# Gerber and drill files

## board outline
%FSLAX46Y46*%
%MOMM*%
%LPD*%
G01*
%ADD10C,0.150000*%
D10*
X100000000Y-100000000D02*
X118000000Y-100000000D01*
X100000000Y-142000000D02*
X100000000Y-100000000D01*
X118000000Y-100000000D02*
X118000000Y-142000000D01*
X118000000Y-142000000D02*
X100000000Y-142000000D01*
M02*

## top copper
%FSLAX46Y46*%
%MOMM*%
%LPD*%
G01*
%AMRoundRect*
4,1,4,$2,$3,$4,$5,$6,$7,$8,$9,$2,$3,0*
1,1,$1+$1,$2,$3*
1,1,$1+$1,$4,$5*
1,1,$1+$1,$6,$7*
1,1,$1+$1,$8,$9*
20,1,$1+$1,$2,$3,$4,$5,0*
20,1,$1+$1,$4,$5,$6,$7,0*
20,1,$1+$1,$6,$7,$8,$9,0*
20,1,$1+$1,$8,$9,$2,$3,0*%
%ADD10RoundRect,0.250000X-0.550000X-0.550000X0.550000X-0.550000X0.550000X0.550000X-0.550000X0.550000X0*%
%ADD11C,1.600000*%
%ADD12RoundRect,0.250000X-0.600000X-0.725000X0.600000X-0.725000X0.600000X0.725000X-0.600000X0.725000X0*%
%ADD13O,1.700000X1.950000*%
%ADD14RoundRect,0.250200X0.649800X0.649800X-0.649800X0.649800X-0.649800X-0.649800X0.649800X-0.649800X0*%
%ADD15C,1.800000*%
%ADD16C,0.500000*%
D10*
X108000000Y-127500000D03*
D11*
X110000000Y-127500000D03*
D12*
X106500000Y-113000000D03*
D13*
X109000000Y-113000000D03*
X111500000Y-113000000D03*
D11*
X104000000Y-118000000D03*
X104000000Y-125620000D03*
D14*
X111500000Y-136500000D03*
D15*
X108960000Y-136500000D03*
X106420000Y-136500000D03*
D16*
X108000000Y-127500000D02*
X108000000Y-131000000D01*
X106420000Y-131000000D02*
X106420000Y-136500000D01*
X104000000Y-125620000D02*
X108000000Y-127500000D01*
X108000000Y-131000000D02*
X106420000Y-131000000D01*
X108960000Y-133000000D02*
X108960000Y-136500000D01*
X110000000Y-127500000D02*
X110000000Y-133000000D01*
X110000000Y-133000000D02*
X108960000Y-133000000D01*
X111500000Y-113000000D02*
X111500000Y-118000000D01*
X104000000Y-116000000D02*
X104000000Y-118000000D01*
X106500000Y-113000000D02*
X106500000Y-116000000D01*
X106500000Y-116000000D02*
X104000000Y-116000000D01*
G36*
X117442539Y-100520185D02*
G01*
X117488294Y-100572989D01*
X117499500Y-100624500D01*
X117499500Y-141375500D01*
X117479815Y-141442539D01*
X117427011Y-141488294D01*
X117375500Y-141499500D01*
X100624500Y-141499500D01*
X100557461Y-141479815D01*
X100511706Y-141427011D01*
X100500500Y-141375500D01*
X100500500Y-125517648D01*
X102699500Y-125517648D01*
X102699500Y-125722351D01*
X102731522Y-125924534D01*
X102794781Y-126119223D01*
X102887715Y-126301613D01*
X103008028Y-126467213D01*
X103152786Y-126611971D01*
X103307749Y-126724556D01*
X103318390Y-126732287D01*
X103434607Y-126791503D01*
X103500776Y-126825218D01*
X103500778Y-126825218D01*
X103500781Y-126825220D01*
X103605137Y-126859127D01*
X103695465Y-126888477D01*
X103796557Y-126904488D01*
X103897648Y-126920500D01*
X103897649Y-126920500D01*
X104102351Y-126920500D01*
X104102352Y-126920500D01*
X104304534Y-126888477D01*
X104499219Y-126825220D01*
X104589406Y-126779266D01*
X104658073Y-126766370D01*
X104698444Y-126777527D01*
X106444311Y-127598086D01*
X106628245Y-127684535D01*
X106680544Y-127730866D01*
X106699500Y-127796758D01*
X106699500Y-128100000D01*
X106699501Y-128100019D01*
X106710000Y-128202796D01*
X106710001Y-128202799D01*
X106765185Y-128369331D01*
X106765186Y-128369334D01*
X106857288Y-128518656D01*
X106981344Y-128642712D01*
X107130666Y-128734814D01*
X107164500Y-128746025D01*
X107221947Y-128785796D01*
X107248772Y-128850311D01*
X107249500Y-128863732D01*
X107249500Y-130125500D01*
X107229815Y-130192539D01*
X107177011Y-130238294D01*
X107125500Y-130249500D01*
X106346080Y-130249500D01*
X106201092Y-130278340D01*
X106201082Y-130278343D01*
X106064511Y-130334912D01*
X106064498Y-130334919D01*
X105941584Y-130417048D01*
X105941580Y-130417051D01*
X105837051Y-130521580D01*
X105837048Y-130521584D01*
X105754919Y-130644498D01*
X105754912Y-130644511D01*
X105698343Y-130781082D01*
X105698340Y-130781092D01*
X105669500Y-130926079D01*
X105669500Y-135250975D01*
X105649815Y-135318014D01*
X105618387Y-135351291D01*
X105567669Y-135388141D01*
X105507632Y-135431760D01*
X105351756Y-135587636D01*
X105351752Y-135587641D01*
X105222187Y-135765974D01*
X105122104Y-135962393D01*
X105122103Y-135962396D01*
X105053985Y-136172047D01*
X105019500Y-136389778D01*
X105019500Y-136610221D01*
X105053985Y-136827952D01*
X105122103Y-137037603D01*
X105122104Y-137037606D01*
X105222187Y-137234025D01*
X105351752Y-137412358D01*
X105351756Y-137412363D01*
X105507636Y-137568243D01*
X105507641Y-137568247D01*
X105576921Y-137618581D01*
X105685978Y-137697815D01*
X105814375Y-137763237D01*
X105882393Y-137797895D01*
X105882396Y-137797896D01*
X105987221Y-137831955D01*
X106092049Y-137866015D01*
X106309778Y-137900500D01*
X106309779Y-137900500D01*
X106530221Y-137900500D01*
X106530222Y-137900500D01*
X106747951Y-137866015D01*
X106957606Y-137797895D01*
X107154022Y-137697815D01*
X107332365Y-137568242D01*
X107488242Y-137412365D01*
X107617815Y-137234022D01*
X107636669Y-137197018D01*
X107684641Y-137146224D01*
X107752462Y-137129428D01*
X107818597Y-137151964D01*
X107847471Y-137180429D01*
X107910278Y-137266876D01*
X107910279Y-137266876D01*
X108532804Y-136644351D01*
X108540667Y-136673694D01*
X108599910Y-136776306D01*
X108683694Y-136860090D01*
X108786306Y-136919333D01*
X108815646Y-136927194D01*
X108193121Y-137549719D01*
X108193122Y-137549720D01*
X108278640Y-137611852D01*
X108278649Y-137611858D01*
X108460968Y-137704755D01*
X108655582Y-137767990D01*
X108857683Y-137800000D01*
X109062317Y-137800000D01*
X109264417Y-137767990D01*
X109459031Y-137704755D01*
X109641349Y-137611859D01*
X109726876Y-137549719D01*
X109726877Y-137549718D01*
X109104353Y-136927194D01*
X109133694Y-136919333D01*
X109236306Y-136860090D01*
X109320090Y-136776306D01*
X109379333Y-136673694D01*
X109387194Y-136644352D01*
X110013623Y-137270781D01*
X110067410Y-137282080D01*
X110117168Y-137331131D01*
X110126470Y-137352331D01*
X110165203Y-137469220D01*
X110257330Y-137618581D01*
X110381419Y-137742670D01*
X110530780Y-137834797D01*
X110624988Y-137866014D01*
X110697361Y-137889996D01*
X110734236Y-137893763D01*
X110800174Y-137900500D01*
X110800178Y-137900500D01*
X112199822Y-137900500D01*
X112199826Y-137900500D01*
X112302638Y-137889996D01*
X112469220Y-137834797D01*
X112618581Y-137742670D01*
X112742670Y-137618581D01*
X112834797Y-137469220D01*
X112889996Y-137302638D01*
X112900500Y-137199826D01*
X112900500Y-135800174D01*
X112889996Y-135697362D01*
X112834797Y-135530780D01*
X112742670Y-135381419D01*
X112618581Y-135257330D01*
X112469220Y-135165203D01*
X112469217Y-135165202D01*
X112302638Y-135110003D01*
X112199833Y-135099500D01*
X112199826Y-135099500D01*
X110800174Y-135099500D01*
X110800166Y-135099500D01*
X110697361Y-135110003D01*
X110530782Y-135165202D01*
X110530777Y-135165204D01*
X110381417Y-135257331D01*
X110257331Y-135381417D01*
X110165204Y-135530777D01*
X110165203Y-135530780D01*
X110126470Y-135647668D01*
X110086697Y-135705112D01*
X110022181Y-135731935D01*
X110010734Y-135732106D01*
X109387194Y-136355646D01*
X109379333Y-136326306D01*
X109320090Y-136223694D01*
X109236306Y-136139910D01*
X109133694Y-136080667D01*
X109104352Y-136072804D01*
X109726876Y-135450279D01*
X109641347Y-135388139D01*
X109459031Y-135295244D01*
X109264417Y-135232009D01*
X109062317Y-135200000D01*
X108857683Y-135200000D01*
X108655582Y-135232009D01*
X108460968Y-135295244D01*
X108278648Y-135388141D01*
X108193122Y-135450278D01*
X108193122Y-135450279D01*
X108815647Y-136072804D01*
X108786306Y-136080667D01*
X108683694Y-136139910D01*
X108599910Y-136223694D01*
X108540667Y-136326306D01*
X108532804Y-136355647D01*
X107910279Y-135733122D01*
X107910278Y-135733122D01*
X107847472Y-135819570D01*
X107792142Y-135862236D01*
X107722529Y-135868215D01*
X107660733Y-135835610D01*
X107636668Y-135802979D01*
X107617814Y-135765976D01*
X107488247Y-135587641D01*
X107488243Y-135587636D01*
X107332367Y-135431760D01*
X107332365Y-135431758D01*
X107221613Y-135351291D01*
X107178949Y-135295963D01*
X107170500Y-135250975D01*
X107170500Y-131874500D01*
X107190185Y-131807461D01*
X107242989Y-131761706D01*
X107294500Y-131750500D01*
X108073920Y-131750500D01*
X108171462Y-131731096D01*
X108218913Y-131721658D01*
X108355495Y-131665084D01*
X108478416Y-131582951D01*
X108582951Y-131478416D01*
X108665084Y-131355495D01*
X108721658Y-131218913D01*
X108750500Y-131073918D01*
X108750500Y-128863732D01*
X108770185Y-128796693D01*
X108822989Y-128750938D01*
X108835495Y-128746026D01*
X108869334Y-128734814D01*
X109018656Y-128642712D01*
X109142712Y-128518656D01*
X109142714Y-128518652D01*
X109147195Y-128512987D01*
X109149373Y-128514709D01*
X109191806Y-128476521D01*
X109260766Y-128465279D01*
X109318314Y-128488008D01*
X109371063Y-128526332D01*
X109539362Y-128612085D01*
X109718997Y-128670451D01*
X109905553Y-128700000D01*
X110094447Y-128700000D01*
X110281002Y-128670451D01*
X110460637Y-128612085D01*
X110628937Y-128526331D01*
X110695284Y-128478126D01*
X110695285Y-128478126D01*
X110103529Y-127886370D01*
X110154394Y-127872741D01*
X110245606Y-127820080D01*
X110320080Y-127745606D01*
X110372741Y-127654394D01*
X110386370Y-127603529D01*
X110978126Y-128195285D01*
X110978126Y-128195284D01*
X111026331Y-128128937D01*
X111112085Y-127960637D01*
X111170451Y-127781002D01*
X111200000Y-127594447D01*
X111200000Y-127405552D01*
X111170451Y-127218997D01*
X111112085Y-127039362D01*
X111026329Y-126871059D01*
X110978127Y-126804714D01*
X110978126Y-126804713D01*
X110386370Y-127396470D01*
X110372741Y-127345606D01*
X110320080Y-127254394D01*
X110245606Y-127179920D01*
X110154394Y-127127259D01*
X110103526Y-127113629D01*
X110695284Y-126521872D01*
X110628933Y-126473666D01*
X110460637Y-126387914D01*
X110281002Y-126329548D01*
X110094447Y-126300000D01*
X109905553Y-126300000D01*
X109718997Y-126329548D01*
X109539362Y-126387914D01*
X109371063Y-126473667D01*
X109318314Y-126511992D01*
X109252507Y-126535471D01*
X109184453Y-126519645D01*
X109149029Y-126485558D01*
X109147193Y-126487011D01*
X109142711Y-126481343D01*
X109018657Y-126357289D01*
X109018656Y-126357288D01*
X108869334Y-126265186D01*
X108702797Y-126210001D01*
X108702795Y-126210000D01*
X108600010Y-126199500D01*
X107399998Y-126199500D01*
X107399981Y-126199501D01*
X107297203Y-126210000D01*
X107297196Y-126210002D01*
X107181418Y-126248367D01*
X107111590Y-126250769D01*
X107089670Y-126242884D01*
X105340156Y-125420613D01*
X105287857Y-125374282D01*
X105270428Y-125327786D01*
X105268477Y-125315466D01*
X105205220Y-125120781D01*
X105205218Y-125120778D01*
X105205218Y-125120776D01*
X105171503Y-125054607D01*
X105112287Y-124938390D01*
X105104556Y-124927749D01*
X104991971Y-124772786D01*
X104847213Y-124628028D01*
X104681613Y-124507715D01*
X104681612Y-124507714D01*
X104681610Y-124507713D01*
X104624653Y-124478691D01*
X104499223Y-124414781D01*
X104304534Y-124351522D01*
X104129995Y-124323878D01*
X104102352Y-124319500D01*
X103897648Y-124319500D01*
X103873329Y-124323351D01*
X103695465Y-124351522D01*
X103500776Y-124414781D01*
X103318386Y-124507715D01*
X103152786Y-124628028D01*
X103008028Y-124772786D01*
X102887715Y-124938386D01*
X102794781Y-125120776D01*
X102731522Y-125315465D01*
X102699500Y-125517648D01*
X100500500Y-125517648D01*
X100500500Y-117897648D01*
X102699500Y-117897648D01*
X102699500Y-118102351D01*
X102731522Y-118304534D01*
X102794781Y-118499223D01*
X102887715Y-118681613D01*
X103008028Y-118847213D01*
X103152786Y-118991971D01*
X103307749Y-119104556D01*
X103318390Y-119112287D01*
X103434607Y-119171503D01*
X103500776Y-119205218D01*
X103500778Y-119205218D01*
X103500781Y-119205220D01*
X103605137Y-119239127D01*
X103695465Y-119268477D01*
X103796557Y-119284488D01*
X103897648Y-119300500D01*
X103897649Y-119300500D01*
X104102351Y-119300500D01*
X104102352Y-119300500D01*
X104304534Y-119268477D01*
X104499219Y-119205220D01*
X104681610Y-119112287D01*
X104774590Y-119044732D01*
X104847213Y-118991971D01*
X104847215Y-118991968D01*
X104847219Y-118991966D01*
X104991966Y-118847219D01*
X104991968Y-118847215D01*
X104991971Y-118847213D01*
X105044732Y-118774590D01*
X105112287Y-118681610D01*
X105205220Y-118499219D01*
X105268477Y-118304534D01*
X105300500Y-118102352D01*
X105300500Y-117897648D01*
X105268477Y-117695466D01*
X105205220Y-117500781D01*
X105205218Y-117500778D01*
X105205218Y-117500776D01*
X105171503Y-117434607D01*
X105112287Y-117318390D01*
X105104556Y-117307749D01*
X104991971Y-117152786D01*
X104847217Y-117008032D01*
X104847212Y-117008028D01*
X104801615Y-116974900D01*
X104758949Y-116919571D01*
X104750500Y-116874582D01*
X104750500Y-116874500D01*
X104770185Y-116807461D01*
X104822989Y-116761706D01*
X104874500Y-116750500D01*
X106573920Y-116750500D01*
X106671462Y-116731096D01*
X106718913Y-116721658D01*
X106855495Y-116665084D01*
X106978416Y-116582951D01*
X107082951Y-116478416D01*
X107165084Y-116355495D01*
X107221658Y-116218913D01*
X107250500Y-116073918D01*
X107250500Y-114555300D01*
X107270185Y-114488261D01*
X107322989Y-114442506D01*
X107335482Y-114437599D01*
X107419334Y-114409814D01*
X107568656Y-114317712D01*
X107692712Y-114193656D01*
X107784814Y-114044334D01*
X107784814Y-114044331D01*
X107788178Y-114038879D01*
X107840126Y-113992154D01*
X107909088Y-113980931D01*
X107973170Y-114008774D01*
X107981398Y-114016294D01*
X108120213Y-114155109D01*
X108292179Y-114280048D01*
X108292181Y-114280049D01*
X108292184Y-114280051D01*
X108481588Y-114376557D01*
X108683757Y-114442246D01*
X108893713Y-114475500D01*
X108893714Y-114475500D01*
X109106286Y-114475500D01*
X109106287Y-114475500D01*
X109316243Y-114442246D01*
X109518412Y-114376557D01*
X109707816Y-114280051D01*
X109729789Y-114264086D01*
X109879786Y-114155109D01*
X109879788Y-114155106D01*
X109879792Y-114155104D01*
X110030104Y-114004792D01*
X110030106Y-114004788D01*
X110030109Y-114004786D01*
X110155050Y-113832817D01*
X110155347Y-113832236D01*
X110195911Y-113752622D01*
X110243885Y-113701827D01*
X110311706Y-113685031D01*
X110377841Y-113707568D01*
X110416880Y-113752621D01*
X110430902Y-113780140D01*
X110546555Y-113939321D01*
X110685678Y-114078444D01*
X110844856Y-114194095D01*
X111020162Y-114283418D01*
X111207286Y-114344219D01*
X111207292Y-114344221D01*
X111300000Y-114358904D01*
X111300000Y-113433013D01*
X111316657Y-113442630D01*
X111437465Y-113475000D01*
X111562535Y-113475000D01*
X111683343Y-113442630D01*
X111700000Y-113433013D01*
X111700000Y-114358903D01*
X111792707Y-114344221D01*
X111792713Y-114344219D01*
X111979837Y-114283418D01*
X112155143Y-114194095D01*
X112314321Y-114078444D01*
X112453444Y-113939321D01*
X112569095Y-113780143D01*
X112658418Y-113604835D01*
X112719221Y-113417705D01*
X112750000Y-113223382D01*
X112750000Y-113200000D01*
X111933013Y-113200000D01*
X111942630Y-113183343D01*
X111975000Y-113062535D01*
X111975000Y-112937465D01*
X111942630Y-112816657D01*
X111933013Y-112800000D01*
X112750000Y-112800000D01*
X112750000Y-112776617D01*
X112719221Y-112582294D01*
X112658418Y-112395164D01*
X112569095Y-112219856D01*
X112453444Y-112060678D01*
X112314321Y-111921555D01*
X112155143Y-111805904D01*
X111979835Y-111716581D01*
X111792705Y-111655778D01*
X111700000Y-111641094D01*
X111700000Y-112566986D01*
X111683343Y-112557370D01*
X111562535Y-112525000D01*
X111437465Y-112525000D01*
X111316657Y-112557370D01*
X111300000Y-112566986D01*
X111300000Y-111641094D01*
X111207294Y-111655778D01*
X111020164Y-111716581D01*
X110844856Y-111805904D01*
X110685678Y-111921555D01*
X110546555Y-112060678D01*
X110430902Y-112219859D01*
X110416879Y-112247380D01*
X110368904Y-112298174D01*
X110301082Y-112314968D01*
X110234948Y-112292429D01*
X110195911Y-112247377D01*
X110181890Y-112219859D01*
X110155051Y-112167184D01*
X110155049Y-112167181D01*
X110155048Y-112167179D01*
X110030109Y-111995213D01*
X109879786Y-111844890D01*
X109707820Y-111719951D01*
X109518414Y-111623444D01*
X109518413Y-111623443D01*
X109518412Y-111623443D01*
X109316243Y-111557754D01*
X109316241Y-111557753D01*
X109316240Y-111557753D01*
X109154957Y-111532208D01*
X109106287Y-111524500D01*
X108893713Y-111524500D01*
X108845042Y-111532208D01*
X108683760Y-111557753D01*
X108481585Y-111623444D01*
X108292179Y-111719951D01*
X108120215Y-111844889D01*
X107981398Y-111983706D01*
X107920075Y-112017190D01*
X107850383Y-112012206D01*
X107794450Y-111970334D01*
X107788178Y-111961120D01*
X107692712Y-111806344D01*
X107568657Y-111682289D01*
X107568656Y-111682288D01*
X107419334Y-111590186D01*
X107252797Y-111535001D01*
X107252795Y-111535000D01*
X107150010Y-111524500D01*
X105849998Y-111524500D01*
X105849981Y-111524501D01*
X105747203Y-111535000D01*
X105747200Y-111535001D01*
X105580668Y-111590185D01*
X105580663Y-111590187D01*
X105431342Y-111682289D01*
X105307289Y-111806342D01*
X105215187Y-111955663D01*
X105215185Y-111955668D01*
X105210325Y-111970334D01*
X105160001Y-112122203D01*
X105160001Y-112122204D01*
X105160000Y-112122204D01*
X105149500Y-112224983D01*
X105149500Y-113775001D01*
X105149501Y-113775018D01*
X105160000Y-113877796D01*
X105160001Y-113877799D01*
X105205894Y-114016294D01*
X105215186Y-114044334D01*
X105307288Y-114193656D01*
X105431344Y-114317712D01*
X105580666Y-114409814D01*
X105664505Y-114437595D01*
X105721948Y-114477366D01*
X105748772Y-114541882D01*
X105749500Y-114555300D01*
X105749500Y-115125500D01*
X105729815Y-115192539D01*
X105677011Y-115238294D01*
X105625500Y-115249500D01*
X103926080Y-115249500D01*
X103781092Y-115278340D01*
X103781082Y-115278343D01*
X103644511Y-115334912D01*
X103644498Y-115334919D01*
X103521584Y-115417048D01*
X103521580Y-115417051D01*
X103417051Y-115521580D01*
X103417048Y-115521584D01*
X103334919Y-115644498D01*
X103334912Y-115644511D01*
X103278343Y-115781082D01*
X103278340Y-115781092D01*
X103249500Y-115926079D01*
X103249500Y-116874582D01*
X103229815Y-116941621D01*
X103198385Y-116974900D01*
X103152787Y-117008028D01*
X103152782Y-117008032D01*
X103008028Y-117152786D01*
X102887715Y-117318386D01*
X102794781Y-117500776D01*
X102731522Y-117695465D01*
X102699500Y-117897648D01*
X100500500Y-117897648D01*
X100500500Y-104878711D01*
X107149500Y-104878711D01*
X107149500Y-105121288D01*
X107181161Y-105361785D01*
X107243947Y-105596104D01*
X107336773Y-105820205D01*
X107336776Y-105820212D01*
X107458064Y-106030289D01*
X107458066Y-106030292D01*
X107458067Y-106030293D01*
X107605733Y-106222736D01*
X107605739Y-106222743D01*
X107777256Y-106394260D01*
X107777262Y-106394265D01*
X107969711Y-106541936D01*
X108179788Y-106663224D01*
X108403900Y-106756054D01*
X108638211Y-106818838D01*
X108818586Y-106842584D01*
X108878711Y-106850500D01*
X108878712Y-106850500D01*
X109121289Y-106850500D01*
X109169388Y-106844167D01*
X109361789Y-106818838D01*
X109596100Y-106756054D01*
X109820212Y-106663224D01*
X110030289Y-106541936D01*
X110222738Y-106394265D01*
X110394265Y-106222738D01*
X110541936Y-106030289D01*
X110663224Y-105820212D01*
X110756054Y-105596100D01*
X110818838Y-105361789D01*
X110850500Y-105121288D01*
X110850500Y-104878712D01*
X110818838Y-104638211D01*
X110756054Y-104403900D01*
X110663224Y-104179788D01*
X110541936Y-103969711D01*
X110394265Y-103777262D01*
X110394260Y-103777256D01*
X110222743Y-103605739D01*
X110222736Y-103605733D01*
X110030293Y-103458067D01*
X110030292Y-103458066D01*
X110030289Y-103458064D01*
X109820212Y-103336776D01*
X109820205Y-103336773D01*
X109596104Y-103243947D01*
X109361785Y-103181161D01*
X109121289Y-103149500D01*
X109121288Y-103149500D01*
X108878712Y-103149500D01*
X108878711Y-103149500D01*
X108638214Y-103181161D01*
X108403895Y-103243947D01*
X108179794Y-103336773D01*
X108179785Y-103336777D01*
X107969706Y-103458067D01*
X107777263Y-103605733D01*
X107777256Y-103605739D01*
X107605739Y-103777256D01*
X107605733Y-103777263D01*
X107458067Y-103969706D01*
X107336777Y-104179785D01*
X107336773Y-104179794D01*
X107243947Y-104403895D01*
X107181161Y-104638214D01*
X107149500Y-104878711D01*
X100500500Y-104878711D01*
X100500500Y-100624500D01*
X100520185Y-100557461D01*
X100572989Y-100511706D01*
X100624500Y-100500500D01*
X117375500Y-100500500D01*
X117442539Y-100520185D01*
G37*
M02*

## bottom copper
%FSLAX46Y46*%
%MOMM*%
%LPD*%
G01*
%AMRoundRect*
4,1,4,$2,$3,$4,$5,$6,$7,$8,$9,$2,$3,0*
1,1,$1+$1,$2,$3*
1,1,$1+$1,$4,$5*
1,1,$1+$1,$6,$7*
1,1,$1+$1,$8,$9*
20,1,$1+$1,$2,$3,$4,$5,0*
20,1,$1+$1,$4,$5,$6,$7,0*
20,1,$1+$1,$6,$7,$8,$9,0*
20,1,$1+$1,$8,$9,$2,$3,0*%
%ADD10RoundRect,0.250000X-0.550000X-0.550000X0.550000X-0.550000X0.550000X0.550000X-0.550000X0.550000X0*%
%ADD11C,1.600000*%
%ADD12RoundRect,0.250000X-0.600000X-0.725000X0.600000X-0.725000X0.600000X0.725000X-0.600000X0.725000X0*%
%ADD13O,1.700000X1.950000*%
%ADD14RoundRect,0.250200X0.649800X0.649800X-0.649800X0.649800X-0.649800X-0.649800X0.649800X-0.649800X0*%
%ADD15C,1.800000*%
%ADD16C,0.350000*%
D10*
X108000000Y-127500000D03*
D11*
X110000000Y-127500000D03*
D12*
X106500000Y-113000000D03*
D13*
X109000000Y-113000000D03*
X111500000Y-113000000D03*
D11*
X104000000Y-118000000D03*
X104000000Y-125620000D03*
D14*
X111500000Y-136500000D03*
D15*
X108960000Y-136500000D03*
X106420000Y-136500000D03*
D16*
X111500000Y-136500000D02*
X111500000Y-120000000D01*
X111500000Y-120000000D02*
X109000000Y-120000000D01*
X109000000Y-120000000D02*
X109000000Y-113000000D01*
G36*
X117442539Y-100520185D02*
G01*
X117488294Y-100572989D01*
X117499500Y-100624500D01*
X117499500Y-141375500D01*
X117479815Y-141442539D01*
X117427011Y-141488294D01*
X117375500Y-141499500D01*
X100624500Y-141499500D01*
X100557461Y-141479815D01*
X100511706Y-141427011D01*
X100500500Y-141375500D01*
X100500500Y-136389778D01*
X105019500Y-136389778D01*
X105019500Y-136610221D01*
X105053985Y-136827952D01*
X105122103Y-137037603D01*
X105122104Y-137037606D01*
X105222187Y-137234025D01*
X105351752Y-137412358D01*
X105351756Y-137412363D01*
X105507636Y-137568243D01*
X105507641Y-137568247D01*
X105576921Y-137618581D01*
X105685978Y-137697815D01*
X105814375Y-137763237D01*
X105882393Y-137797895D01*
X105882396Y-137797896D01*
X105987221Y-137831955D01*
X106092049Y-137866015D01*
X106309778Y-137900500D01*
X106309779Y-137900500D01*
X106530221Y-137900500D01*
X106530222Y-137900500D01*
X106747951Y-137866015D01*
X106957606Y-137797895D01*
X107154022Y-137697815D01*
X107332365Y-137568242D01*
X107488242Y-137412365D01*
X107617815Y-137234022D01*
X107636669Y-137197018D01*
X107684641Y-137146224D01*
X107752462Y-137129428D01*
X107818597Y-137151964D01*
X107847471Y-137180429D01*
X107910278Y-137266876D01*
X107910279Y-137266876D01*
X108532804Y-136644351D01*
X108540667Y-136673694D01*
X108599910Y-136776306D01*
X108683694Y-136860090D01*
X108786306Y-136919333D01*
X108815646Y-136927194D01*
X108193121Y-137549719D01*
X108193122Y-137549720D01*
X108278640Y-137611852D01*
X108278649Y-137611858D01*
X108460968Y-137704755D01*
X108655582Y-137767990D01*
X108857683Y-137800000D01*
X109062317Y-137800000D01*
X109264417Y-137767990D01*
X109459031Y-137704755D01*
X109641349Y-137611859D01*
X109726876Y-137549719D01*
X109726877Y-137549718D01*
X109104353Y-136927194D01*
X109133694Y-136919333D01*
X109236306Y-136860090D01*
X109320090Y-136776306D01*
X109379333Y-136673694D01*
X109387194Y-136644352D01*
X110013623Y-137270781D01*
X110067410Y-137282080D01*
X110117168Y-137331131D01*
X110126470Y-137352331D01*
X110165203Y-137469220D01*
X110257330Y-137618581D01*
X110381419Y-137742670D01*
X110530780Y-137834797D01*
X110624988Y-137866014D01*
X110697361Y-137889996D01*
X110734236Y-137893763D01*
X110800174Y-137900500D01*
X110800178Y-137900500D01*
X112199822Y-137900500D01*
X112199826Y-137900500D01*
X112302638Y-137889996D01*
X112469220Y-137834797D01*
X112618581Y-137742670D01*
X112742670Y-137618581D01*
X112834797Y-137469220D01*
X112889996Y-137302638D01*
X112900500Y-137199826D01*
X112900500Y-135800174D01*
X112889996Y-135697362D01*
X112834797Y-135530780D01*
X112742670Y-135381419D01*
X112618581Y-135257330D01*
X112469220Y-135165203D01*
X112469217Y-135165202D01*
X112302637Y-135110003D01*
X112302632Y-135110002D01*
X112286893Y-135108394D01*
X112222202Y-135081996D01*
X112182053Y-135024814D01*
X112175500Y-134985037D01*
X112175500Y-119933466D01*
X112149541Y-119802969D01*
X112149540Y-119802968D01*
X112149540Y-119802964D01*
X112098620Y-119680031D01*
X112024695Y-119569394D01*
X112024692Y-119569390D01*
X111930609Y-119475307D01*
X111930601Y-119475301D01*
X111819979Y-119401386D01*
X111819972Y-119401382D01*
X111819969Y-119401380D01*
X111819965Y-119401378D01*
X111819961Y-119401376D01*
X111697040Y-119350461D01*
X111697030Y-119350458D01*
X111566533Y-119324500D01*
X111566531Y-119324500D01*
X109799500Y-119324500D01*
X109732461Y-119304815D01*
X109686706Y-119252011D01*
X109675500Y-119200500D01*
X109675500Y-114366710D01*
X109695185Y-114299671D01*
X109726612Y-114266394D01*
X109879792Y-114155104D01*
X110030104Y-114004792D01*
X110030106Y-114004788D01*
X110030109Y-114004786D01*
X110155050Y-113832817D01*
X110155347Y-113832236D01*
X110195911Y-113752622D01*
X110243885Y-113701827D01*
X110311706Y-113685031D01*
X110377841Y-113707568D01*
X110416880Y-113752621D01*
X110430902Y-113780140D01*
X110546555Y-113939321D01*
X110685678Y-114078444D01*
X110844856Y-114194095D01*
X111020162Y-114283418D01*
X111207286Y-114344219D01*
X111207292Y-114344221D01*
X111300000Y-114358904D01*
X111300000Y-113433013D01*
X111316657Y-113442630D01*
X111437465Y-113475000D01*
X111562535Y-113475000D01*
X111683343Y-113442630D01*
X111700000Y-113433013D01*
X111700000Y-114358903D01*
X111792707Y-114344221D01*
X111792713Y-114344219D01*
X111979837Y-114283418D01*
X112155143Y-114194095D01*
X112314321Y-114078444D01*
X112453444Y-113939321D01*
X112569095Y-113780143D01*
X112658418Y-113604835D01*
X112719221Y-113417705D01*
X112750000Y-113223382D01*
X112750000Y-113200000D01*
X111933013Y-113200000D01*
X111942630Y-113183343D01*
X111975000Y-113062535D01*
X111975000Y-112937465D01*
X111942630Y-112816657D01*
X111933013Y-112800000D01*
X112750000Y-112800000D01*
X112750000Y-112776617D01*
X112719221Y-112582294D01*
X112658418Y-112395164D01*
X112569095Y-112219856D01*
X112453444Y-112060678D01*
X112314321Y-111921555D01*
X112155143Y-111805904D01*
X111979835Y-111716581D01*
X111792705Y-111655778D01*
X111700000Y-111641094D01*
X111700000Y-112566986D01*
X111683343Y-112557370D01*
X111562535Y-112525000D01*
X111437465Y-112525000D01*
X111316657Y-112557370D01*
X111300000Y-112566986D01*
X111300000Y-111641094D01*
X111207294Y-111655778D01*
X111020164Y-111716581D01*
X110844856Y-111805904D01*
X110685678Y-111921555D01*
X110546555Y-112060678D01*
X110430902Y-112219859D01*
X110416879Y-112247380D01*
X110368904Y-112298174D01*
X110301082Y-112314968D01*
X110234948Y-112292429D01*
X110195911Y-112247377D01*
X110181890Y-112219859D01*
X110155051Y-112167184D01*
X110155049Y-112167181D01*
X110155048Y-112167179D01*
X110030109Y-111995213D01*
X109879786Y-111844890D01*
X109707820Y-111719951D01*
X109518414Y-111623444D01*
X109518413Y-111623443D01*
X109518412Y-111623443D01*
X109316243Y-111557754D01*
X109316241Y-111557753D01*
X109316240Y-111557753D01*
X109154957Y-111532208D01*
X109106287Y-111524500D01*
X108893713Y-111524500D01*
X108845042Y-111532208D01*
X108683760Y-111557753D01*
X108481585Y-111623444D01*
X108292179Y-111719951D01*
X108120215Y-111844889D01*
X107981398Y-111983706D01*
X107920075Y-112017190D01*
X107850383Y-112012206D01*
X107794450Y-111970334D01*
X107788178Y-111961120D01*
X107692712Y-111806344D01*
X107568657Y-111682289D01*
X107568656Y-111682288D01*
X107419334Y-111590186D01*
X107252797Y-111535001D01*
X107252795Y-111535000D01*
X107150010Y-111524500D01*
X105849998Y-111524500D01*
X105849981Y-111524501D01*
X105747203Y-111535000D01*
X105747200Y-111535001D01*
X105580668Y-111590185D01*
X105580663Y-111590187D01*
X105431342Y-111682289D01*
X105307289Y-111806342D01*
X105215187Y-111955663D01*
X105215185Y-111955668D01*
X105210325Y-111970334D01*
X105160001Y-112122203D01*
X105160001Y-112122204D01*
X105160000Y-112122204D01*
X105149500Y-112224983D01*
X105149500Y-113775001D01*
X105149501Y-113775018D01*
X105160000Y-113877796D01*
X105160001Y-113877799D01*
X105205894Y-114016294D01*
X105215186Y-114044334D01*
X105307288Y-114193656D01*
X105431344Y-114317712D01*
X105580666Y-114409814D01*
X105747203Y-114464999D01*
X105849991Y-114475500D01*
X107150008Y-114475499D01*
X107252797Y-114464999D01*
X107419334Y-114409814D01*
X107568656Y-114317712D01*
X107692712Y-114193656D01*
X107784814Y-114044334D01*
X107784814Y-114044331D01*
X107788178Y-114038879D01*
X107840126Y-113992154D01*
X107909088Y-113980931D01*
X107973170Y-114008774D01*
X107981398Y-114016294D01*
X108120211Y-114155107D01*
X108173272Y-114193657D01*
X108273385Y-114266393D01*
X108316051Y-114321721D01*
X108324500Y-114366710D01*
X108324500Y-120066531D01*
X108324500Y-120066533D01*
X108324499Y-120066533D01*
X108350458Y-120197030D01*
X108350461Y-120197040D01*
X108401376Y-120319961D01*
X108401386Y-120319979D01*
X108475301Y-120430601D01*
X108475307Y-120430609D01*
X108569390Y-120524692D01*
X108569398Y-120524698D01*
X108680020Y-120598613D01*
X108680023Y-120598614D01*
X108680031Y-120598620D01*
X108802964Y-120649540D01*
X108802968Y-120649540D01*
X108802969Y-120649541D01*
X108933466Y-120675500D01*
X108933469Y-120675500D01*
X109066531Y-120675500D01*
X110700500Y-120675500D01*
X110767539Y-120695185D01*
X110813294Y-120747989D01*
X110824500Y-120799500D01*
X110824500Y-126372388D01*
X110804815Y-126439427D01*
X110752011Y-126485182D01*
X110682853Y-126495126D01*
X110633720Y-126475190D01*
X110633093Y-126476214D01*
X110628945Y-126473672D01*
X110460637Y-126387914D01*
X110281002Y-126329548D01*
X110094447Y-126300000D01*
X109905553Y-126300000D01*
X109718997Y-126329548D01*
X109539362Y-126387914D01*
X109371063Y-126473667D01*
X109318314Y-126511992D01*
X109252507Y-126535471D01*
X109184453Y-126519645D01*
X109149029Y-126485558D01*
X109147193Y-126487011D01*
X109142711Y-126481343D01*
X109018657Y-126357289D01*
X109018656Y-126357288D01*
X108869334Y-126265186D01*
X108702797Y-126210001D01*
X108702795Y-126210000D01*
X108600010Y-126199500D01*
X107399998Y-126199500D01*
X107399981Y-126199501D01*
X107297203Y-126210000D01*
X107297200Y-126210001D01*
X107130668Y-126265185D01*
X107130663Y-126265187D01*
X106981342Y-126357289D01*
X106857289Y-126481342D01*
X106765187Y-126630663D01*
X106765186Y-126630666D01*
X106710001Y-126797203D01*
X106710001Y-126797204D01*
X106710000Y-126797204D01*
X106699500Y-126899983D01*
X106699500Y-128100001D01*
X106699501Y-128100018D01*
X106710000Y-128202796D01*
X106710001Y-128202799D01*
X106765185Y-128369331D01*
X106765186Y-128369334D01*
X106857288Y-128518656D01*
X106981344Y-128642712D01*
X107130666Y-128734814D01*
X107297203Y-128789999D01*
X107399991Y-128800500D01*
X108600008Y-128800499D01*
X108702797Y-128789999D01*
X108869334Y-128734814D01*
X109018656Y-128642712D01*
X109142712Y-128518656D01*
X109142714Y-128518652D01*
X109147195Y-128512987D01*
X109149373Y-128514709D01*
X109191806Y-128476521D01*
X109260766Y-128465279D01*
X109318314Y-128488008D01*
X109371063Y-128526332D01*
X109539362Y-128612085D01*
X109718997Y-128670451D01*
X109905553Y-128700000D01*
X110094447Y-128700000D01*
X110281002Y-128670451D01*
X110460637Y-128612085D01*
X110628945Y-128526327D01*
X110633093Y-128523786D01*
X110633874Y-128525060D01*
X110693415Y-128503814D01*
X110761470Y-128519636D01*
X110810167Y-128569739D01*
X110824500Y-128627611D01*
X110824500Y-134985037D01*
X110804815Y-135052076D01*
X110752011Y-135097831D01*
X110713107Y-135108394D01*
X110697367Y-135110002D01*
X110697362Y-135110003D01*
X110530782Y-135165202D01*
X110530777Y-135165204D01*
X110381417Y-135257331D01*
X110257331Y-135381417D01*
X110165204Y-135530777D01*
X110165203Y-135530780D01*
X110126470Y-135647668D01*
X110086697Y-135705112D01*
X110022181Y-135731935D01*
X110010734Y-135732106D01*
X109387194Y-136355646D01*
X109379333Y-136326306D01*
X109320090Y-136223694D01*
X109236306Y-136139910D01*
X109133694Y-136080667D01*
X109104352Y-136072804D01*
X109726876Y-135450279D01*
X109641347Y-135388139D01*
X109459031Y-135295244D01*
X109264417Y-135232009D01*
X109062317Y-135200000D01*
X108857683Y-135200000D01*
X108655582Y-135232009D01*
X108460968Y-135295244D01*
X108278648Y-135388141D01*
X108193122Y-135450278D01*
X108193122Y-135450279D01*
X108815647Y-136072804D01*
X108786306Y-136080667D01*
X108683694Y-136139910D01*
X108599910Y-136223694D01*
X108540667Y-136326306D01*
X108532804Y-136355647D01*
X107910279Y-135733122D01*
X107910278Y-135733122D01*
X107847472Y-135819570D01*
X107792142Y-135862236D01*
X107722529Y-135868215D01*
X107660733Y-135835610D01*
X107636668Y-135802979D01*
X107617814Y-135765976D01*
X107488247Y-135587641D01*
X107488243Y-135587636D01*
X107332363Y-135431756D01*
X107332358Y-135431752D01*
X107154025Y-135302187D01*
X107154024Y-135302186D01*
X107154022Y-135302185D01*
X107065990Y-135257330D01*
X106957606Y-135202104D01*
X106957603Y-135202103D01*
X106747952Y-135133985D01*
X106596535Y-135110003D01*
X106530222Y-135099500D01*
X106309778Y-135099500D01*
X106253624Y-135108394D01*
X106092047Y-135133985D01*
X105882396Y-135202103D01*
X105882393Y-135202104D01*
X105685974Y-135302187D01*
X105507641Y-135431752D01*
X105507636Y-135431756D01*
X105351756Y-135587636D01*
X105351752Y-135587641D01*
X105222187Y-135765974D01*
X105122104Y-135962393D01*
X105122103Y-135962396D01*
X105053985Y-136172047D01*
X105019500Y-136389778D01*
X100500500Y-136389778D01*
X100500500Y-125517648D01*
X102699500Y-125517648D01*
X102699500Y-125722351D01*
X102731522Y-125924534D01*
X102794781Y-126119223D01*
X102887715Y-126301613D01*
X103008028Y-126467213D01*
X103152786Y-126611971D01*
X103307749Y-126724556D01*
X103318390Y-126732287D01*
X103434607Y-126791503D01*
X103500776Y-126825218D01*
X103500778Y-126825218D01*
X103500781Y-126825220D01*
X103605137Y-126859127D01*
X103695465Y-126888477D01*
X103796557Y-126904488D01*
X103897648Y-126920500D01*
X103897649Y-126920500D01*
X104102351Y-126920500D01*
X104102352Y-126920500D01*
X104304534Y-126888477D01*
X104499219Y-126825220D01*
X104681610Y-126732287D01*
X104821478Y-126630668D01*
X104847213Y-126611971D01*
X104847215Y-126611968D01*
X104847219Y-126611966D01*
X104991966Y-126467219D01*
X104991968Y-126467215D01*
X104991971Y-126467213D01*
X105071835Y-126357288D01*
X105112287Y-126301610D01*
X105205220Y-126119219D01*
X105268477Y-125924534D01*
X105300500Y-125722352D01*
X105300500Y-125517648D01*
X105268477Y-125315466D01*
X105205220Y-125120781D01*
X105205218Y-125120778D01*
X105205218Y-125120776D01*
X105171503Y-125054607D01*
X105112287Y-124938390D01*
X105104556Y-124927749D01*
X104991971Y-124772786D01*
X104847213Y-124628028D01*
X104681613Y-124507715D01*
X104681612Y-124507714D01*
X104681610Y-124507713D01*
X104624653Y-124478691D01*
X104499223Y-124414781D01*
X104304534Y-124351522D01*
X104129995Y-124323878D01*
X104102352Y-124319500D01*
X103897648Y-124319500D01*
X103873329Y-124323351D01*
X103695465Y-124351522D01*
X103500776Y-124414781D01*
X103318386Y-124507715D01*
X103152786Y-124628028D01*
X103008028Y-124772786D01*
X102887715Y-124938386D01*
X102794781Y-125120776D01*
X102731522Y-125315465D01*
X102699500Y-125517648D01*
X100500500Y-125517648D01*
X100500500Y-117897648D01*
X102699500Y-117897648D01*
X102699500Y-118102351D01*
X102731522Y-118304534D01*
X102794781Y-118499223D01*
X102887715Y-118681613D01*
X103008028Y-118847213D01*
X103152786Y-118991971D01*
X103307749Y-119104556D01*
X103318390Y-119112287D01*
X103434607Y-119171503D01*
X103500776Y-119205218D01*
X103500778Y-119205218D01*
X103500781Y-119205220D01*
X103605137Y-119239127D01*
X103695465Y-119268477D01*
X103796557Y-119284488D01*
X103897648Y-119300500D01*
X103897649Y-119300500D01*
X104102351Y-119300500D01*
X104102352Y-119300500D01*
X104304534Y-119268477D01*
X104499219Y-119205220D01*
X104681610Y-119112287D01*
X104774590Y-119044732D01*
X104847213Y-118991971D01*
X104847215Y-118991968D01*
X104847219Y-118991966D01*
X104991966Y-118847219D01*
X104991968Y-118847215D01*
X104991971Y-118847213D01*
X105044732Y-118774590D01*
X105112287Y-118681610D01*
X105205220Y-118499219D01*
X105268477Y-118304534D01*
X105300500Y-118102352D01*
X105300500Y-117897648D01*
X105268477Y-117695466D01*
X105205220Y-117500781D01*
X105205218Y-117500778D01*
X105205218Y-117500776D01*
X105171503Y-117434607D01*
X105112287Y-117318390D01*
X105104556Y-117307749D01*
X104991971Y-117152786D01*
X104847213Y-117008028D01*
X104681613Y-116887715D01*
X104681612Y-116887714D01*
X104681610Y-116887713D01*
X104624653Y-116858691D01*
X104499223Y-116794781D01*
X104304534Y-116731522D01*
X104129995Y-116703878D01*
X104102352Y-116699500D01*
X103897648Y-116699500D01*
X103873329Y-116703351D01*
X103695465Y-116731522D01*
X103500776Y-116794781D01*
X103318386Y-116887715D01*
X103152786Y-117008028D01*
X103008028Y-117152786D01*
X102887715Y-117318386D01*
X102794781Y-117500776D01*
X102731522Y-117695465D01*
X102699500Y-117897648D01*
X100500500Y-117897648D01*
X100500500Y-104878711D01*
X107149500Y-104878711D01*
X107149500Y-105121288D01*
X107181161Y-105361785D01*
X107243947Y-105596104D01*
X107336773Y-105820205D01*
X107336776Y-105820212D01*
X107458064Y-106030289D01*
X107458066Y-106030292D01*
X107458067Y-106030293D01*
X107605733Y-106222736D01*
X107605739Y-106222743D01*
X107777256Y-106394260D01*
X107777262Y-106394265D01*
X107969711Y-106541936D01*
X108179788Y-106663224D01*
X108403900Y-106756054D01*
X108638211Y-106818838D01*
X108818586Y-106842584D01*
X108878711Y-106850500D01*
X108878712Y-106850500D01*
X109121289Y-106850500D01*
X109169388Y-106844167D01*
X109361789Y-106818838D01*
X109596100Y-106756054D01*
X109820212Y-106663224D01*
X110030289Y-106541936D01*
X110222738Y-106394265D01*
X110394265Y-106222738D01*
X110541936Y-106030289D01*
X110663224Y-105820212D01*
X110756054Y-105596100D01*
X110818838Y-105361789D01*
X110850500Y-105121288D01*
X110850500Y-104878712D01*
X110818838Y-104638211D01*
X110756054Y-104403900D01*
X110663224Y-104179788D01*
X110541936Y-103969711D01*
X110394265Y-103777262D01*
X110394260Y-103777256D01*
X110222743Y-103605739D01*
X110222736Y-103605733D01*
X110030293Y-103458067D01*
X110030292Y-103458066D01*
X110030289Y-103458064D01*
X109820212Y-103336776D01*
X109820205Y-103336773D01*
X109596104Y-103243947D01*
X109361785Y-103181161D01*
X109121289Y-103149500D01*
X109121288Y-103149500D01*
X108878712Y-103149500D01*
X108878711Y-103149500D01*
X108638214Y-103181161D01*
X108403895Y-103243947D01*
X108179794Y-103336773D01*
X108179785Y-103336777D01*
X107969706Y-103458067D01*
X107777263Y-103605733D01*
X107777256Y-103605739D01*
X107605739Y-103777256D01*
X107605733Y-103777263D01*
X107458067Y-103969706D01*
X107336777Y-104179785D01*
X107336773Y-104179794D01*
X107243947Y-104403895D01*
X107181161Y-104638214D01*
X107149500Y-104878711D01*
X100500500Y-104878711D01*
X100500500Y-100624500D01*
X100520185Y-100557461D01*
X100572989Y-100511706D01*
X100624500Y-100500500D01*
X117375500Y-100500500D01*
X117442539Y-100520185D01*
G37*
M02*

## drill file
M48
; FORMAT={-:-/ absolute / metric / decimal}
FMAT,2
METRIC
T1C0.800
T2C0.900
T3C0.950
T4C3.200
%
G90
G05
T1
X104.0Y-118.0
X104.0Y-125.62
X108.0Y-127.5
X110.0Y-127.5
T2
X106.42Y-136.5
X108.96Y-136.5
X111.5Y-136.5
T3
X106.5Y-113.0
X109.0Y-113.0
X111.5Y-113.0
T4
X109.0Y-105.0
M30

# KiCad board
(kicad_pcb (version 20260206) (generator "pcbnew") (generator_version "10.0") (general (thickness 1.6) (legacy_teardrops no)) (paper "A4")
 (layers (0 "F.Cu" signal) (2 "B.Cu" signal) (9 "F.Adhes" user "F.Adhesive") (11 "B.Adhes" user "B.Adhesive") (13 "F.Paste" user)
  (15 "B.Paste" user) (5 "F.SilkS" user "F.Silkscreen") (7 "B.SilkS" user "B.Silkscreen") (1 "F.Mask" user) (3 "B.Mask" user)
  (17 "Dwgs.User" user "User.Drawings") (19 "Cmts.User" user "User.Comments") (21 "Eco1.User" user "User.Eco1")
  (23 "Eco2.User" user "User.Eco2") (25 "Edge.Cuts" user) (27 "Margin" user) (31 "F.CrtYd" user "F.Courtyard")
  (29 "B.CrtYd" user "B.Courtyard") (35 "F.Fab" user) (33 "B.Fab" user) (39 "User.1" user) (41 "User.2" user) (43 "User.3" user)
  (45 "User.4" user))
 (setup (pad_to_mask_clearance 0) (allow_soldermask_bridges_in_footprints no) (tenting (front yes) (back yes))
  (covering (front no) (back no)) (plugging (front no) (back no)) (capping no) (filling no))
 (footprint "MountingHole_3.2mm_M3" (layer "F.Cu") (at 109 105)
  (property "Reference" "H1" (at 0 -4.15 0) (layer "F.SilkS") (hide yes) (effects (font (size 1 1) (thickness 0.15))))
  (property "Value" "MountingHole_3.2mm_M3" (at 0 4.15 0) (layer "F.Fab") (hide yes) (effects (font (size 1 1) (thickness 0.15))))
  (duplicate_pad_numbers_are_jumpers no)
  (pad "" np_thru_hole circle (at 0 0) (size 3.2 3.2) (drill 3.2) (layers "*.Cu" "*.Mask")))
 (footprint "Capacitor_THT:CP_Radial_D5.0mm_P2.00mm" (layer "F.Cu") (at 108 127.5)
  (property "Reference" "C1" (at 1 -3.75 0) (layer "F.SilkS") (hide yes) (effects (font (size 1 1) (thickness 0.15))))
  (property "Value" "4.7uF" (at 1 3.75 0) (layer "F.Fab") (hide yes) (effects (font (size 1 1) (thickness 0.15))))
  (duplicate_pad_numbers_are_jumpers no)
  (pad "1" thru_hole roundrect (at 0 0) (size 1.6 1.6) (drill 0.8) (layers "*.Cu" "*.Mask") (remove_unused_layers no)
   (roundrect_rratio 0.15625) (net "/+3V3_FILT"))
  (pad "2" thru_hole circle (at 2 0) (size 1.6 1.6) (drill 0.8) (layers "*.Cu" "*.Mask") (remove_unused_layers no) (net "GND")))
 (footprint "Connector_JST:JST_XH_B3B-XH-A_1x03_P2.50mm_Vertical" (layer "F.Cu") (at 106.5 113)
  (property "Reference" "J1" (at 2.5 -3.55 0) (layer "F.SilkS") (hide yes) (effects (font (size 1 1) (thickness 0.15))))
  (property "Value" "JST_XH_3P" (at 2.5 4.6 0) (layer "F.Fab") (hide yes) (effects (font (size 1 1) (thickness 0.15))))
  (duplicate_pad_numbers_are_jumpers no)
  (pad "1" thru_hole roundrect (at 0 0) (size 1.7 1.95) (drill 0.95) (layers "*.Cu" "*.Mask") (remove_unused_layers no)
   (roundrect_rratio 0.147059) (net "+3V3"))
  (pad "2" thru_hole oval (at 2.5 0) (size 1.7 1.95) (drill 0.95) (layers "*.Cu" "*.Mask") (remove_unused_layers no) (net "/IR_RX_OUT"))
  (pad "3" thru_hole oval (at 5 0) (size 1.7 1.95) (drill 0.95) (layers "*.Cu" "*.Mask") (remove_unused_layers no) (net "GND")))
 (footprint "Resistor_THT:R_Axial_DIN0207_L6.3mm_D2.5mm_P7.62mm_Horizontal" (layer "F.Cu") (at 104 118 -90)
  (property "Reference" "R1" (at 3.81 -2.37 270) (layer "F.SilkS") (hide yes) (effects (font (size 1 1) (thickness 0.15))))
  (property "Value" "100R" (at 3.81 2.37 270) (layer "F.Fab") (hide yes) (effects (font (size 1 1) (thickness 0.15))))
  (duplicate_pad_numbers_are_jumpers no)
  (pad "1" thru_hole circle (at 0 0 270) (size 1.6 1.6) (drill 0.8) (layers "*.Cu" "*.Mask") (remove_unused_layers no) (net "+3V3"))
  (pad "2" thru_hole circle (at 7.62 0 270) (size 1.6 1.6) (drill 0.8) (layers "*.Cu" "*.Mask") (remove_unused_layers no) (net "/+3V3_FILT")))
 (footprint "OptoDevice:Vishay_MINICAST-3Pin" (layer "F.Cu") (at 111.5 136.5 180)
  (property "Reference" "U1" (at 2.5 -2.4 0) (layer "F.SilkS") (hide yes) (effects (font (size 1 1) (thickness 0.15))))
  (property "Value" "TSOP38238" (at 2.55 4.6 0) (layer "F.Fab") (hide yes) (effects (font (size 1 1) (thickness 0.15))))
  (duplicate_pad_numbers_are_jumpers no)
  (pad "1" thru_hole roundrect (at 0 0 180) (size 1.8 1.8) (drill 0.9) (layers "*.Cu" "*.Mask") (remove_unused_layers no)
   (roundrect_rratio 0.139) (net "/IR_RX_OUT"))
  (pad "2" thru_hole circle (at 2.54 0 180) (size 1.8 1.8) (drill 0.9) (layers "*.Cu" "*.Mask") (remove_unused_layers no) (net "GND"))
  (pad "3" thru_hole circle (at 5.08 0 180) (size 1.8 1.8) (drill 0.9) (layers "*.Cu" "*.Mask") (remove_unused_layers no) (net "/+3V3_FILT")))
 (gr_line (start 100 100) (end 118 100) (stroke (width 0.15) (type default)) (layer "Edge.Cuts"))
 (gr_line (start 100 142) (end 100 100) (stroke (width 0.15) (type default)) (layer "Edge.Cuts"))
 (gr_line (start 118 100) (end 118 142) (stroke (width 0.15) (type default)) (layer "Edge.Cuts"))
 (gr_line (start 118 142) (end 100 142) (stroke (width 0.15) (type default)) (layer "Edge.Cuts"))
 (segment (start 108 127.5) (end 108 131) (width 0.5) (layer "F.Cu") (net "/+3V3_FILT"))
 (segment (start 106.42 131) (end 106.42 136.5) (width 0.5) (layer "F.Cu") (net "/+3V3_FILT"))
 (segment (start 104 125.62) (end 108 127.5) (width 0.5) (layer "F.Cu") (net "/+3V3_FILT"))
 (segment (start 108 131) (end 106.42 131) (width 0.5) (layer "F.Cu") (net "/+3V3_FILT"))
 (segment (start 108.96 133) (end 108.96 136.5) (width 0.5) (layer "F.Cu") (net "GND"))
 (segment (start 110 127.5) (end 110 133) (width 0.5) (layer "F.Cu") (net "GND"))
 (segment (start 110 133) (end 108.96 133) (width 0.5) (layer "F.Cu") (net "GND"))
 (segment (start 111.5 113) (end 111.5 118) (width 0.5) (layer "F.Cu") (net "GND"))
 (segment (start 104 116) (end 104 118) (width 0.5) (layer "F.Cu") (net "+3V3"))
 (segment (start 106.5 113) (end 106.5 116) (width 0.5) (layer "F.Cu") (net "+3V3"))
 (segment (start 106.5 116) (end 104 116) (width 0.5) (layer "F.Cu") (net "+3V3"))
 (segment (start 111.5 136.5) (end 111.5 120) (width 0.35) (layer "B.Cu") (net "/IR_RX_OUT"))
 (segment (start 111.5 120) (end 109 120) (width 0.35) (layer "B.Cu") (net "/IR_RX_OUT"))
 (segment (start 109 120) (end 109 113) (width 0.35) (layer "B.Cu") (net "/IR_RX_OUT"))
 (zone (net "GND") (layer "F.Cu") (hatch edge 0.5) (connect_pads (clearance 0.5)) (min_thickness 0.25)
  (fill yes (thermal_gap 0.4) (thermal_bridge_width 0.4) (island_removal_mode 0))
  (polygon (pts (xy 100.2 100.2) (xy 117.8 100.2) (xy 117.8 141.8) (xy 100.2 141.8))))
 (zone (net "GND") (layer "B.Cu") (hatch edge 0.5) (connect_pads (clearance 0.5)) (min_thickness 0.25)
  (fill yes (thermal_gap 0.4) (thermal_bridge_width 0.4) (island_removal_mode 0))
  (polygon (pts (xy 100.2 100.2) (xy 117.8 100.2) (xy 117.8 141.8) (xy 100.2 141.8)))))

